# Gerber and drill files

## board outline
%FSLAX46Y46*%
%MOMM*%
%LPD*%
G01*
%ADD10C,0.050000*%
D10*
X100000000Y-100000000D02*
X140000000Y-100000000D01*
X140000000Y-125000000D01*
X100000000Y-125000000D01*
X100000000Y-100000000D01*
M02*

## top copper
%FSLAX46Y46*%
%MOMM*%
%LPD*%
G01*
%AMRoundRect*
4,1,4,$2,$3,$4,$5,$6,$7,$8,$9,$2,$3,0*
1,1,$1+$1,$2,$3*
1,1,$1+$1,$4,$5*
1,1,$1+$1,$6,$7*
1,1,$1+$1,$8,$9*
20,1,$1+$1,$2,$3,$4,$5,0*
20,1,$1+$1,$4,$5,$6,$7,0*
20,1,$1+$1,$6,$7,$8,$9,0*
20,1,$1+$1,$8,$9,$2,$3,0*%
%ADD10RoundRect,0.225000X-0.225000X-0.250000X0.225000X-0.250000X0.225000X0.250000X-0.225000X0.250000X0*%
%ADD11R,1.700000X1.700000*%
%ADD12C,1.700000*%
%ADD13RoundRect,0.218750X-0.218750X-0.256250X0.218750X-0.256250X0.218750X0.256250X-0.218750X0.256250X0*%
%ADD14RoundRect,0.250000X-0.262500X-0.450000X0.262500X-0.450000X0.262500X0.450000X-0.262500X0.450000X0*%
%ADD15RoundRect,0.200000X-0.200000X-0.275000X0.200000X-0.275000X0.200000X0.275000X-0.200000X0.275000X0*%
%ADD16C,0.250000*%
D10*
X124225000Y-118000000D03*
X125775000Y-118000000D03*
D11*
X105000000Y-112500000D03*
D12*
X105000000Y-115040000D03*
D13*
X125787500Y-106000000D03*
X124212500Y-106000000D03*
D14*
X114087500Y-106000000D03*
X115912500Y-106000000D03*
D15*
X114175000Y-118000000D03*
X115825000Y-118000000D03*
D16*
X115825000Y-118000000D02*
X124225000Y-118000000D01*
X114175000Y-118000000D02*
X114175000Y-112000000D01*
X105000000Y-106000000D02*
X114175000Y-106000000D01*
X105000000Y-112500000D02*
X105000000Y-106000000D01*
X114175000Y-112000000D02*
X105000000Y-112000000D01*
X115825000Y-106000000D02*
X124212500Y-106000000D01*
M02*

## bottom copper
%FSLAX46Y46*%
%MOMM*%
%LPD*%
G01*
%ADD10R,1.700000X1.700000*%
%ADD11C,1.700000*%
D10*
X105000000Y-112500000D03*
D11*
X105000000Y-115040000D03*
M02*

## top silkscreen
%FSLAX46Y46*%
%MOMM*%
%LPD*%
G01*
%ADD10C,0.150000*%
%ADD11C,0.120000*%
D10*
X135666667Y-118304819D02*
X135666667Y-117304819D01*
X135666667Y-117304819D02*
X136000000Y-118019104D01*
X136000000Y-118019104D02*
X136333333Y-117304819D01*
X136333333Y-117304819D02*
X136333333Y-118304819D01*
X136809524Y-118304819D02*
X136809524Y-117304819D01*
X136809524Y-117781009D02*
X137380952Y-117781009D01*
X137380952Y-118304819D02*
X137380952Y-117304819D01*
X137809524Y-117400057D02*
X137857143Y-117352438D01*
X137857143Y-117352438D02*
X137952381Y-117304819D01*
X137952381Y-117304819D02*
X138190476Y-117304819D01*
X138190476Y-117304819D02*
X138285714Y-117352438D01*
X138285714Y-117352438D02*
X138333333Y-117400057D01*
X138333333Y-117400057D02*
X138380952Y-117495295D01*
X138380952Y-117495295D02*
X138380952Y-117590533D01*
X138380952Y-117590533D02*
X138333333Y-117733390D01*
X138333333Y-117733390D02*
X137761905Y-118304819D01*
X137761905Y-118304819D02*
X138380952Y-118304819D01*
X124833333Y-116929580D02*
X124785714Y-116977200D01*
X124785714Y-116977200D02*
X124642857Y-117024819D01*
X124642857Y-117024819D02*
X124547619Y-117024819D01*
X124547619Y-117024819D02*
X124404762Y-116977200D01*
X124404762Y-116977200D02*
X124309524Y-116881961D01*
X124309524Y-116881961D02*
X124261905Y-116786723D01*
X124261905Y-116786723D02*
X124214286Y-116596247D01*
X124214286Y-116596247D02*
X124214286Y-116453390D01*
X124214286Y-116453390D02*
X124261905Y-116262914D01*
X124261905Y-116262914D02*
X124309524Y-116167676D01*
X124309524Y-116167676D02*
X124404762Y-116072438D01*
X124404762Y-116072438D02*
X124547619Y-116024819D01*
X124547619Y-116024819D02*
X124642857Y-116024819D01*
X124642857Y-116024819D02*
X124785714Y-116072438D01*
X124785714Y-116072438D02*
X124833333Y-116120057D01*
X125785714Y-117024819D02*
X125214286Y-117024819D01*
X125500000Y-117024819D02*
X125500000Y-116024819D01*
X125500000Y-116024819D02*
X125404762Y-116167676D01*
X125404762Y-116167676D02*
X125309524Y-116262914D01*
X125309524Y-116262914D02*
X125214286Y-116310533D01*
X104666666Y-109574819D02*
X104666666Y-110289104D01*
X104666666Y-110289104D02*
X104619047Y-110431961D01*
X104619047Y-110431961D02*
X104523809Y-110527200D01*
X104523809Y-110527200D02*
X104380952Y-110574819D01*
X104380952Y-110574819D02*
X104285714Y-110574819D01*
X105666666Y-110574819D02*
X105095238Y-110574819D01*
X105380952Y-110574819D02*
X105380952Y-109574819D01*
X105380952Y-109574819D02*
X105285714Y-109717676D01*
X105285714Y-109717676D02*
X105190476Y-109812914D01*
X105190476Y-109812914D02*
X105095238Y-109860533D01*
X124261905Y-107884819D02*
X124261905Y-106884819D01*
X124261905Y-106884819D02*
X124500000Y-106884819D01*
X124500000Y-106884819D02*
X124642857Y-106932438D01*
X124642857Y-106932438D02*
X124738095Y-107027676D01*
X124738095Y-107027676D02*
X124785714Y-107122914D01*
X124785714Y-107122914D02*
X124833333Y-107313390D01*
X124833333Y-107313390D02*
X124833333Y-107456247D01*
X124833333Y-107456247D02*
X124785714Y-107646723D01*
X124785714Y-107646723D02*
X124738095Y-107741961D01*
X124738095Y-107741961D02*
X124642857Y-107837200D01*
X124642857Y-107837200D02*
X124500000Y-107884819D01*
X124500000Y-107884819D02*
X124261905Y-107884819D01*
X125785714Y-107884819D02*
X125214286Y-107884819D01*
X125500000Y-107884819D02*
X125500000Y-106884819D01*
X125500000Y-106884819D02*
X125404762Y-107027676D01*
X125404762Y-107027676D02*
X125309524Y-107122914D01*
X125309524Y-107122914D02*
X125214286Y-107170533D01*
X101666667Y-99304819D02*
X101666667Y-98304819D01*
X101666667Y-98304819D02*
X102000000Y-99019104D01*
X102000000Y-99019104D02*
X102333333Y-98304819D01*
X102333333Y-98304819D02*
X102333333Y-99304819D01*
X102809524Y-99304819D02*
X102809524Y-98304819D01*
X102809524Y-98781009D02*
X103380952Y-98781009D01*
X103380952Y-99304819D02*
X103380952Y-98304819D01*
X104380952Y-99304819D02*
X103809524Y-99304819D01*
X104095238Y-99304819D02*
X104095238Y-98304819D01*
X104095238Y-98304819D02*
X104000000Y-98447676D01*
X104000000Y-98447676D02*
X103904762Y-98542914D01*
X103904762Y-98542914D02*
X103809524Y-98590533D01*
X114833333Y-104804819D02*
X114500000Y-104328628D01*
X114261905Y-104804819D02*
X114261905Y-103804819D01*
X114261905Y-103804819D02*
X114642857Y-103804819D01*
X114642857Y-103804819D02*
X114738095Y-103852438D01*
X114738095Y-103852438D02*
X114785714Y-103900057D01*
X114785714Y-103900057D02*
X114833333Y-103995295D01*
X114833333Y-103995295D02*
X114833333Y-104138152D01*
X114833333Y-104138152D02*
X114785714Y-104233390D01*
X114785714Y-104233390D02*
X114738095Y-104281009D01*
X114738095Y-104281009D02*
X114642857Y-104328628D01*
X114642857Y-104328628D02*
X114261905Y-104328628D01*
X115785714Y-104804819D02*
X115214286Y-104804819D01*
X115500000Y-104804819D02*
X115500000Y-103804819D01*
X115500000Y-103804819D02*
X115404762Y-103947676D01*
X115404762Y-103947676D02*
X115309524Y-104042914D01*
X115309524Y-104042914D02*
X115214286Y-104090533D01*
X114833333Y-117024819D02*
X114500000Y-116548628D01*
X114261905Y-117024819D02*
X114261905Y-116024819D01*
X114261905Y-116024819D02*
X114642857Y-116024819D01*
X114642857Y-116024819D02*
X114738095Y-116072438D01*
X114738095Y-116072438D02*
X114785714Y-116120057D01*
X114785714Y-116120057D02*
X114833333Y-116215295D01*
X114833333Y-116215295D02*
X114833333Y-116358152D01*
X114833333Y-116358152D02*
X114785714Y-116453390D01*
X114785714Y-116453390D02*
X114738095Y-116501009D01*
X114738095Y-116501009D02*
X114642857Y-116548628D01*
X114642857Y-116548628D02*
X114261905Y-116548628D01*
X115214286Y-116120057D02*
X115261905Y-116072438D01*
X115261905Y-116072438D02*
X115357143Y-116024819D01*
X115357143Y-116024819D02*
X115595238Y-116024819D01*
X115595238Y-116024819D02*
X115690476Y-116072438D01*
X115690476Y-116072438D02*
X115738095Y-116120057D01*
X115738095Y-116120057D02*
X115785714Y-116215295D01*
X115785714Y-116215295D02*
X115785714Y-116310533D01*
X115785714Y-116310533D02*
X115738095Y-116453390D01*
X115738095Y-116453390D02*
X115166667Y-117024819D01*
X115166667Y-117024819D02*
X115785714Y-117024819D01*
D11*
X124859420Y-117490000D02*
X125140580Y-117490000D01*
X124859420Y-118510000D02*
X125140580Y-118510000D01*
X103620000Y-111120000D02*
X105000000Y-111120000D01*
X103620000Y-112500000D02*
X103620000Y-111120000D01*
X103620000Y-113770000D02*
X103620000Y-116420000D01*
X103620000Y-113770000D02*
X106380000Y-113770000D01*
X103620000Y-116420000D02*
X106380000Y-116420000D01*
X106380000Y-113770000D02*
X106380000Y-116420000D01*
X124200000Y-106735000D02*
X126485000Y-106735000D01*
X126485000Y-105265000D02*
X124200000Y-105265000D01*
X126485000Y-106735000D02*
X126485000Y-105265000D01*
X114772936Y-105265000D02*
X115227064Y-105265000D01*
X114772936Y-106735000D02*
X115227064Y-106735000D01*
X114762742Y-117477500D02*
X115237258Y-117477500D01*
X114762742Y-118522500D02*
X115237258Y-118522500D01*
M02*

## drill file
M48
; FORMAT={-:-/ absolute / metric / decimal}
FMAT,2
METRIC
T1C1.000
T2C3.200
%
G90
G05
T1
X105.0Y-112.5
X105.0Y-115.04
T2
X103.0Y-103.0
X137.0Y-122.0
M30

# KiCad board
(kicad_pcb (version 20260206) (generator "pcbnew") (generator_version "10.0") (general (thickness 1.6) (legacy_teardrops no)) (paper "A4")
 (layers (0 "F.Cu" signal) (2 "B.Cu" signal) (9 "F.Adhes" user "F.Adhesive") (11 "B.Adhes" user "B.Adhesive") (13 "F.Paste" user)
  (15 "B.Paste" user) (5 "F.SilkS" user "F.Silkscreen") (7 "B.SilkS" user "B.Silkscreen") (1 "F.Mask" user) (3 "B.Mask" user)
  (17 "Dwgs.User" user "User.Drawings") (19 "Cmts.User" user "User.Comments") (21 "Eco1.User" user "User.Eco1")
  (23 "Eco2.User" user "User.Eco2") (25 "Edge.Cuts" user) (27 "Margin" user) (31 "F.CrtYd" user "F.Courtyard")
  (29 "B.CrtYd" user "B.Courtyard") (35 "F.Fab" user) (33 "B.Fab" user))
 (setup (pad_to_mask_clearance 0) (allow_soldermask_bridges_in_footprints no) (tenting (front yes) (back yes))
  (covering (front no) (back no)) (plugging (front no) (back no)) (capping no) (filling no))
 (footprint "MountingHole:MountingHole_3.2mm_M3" (layer "F.Cu") (at 137 122)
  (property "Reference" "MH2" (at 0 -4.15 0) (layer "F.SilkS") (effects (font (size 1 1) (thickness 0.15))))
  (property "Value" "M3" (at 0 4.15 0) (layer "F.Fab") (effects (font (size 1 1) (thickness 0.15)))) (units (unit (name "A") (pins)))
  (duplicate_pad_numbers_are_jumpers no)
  (pad "" np_thru_hole circle (at 0 0) (size 3.2 3.2) (drill 3.2) (layers "*.Cu" "*.Mask")))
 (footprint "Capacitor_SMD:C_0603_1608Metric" (layer "F.Cu") (at 125 118)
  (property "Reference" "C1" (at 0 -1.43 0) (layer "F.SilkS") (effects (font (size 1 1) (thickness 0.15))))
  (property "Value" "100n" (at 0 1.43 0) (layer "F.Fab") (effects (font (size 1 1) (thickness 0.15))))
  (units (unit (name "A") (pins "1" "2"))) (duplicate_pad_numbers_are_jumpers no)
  (fp_line (start -0.14058 -0.51) (end 0.14058 -0.51) (stroke (width 0.12) (type solid)) (layer "F.SilkS"))
  (fp_line (start -0.14058 0.51) (end 0.14058 0.51) (stroke (width 0.12) (type solid)) (layer "F.SilkS"))
  (pad "1" smd roundrect (at -0.775 0) (size 0.9 0.95) (layers "F.Cu" "F.Mask" "F.Paste") (roundrect_rratio 0.25) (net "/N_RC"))
  (pad "2" smd roundrect (at 0.775 0) (size 0.9 0.95) (layers "F.Cu" "F.Mask" "F.Paste") (roundrect_rratio 0.25) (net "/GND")))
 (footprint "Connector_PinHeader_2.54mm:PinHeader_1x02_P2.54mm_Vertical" (layer "F.Cu") (at 105 112.5)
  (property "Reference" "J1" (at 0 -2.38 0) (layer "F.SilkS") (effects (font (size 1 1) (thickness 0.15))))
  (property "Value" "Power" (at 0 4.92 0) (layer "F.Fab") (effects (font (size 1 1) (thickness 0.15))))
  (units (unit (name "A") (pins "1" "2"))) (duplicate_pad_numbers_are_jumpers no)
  (fp_line (start -1.38 -1.38) (end 0 -1.38) (stroke (width 0.12) (type solid)) (layer "F.SilkS"))
  (fp_line (start -1.38 0) (end -1.38 -1.38) (stroke (width 0.12) (type solid)) (layer "F.SilkS"))
  (fp_line (start -1.38 1.27) (end -1.38 3.92) (stroke (width 0.12) (type solid)) (layer "F.SilkS"))
  (fp_line (start -1.38 1.27) (end 1.38 1.27) (stroke (width 0.12) (type solid)) (layer "F.SilkS"))
  (fp_line (start -1.38 3.92) (end 1.38 3.92) (stroke (width 0.12) (type solid)) (layer "F.SilkS"))
  (fp_line (start 1.38 1.27) (end 1.38 3.92) (stroke (width 0.12) (type solid)) (layer "F.SilkS"))
  (pad "1" thru_hole rect (at 0 0) (size 1.7 1.7) (drill 1) (layers "*.Cu" "*.Mask") (remove_unused_layers no) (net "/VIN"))
  (pad "2" thru_hole circle (at 0 2.54) (size 1.7 1.7) (drill 1) (layers "*.Cu" "*.Mask") (remove_unused_layers no) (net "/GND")))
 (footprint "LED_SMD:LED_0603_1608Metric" (layer "F.Cu") (at 125 106 180)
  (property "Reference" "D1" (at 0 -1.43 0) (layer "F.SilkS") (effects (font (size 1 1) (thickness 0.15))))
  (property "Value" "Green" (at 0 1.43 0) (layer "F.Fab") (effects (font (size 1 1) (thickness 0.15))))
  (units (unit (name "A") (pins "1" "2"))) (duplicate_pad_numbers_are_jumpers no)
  (fp_line (start 0.8 -0.735) (end -1.485 -0.735) (stroke (width 0.12) (type solid)) (layer "F.SilkS"))
  (fp_line (start -1.485 0.735) (end 0.8 0.735) (stroke (width 0.12) (type solid)) (layer "F.SilkS"))
  (fp_line (start -1.485 -0.735) (end -1.485 0.735) (stroke (width 0.12) (type solid)) (layer "F.SilkS"))
  (pad "1" smd roundrect (at -0.7875 0) (size 0.875 0.95) (layers "F.Cu" "F.Mask" "F.Paste") (roundrect_rratio 0.25) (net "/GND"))
  (pad "2" smd roundrect (at 0.7875 0) (size 0.875 0.95) (layers "F.Cu" "F.Mask" "F.Paste") (roundrect_rratio 0.25) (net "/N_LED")))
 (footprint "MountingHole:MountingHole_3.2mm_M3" (layer "F.Cu") (at 103 103)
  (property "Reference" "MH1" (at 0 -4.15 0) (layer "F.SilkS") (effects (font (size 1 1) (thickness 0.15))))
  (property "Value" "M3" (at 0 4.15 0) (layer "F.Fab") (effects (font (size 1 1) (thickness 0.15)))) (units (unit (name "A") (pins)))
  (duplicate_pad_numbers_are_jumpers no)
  (pad "" np_thru_hole circle (at 0 0) (size 3.2 3.2) (drill 3.2) (layers "*.Cu" "*.Mask")))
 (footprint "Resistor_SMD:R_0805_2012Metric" (layer "F.Cu") (at 115 106)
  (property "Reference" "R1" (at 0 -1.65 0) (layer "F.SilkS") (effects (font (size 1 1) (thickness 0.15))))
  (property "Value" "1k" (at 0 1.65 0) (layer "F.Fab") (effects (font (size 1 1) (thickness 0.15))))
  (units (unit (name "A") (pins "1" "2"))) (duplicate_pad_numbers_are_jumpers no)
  (fp_line (start -0.227064 -0.735) (end 0.227064 -0.735) (stroke (width 0.12) (type solid)) (layer "F.SilkS"))
  (fp_line (start -0.227064 0.735) (end 0.227064 0.735) (stroke (width 0.12) (type solid)) (layer "F.SilkS"))
  (pad "1" smd roundrect (at -0.9125 0) (size 1.025 1.4) (layers "F.Cu" "F.Mask" "F.Paste") (roundrect_rratio 0.243902) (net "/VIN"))
  (pad "2" smd roundrect (at 0.9125 0) (size 1.025 1.4) (layers "F.Cu" "F.Mask" "F.Paste") (roundrect_rratio 0.243902) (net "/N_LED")))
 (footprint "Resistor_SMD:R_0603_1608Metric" (layer "F.Cu") (at 115 118)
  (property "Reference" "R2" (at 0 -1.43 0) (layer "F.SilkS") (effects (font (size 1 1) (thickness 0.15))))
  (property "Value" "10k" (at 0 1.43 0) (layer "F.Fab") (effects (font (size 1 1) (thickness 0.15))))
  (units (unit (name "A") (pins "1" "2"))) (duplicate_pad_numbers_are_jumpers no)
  (fp_line (start -0.237258 -0.5225) (end 0.237258 -0.5225) (stroke (width 0.12) (type solid)) (layer "F.SilkS"))
  (fp_line (start -0.237258 0.5225) (end 0.237258 0.5225) (stroke (width 0.12) (type solid)) (layer "F.SilkS"))
  (pad "1" smd roundrect (at -0.825 0) (size 0.8 0.95) (layers "F.Cu" "F.Mask" "F.Paste") (roundrect_rratio 0.25) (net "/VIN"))
  (pad "2" smd roundrect (at 0.825 0) (size 0.8 0.95) (layers "F.Cu" "F.Mask" "F.Paste") (roundrect_rratio 0.25) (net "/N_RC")))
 (gr_rect (start 100 100) (end 140 125) (stroke (width 0.05) (type default)) (fill no) (layer "Edge.Cuts"))
 (segment (start 115.825 118) (end 124.225 118) (width 0.25) (layer "F.Cu") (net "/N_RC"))
 (segment (start 114.175 118) (end 114.175 112) (width 0.25) (layer "F.Cu") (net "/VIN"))
 (segment (start 105 106) (end 114.175 106) (width 0.25) (layer "F.Cu") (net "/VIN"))
 (segment (start 105 112.5) (end 105 106) (width 0.25) (layer "F.Cu") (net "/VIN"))
 (segment (start 114.175 112) (end 105 112) (width 0.25) (layer "F.Cu") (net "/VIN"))
 (segment (start 115.825 106) (end 124.2125 106) (width 0.25) (layer "F.Cu") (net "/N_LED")))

